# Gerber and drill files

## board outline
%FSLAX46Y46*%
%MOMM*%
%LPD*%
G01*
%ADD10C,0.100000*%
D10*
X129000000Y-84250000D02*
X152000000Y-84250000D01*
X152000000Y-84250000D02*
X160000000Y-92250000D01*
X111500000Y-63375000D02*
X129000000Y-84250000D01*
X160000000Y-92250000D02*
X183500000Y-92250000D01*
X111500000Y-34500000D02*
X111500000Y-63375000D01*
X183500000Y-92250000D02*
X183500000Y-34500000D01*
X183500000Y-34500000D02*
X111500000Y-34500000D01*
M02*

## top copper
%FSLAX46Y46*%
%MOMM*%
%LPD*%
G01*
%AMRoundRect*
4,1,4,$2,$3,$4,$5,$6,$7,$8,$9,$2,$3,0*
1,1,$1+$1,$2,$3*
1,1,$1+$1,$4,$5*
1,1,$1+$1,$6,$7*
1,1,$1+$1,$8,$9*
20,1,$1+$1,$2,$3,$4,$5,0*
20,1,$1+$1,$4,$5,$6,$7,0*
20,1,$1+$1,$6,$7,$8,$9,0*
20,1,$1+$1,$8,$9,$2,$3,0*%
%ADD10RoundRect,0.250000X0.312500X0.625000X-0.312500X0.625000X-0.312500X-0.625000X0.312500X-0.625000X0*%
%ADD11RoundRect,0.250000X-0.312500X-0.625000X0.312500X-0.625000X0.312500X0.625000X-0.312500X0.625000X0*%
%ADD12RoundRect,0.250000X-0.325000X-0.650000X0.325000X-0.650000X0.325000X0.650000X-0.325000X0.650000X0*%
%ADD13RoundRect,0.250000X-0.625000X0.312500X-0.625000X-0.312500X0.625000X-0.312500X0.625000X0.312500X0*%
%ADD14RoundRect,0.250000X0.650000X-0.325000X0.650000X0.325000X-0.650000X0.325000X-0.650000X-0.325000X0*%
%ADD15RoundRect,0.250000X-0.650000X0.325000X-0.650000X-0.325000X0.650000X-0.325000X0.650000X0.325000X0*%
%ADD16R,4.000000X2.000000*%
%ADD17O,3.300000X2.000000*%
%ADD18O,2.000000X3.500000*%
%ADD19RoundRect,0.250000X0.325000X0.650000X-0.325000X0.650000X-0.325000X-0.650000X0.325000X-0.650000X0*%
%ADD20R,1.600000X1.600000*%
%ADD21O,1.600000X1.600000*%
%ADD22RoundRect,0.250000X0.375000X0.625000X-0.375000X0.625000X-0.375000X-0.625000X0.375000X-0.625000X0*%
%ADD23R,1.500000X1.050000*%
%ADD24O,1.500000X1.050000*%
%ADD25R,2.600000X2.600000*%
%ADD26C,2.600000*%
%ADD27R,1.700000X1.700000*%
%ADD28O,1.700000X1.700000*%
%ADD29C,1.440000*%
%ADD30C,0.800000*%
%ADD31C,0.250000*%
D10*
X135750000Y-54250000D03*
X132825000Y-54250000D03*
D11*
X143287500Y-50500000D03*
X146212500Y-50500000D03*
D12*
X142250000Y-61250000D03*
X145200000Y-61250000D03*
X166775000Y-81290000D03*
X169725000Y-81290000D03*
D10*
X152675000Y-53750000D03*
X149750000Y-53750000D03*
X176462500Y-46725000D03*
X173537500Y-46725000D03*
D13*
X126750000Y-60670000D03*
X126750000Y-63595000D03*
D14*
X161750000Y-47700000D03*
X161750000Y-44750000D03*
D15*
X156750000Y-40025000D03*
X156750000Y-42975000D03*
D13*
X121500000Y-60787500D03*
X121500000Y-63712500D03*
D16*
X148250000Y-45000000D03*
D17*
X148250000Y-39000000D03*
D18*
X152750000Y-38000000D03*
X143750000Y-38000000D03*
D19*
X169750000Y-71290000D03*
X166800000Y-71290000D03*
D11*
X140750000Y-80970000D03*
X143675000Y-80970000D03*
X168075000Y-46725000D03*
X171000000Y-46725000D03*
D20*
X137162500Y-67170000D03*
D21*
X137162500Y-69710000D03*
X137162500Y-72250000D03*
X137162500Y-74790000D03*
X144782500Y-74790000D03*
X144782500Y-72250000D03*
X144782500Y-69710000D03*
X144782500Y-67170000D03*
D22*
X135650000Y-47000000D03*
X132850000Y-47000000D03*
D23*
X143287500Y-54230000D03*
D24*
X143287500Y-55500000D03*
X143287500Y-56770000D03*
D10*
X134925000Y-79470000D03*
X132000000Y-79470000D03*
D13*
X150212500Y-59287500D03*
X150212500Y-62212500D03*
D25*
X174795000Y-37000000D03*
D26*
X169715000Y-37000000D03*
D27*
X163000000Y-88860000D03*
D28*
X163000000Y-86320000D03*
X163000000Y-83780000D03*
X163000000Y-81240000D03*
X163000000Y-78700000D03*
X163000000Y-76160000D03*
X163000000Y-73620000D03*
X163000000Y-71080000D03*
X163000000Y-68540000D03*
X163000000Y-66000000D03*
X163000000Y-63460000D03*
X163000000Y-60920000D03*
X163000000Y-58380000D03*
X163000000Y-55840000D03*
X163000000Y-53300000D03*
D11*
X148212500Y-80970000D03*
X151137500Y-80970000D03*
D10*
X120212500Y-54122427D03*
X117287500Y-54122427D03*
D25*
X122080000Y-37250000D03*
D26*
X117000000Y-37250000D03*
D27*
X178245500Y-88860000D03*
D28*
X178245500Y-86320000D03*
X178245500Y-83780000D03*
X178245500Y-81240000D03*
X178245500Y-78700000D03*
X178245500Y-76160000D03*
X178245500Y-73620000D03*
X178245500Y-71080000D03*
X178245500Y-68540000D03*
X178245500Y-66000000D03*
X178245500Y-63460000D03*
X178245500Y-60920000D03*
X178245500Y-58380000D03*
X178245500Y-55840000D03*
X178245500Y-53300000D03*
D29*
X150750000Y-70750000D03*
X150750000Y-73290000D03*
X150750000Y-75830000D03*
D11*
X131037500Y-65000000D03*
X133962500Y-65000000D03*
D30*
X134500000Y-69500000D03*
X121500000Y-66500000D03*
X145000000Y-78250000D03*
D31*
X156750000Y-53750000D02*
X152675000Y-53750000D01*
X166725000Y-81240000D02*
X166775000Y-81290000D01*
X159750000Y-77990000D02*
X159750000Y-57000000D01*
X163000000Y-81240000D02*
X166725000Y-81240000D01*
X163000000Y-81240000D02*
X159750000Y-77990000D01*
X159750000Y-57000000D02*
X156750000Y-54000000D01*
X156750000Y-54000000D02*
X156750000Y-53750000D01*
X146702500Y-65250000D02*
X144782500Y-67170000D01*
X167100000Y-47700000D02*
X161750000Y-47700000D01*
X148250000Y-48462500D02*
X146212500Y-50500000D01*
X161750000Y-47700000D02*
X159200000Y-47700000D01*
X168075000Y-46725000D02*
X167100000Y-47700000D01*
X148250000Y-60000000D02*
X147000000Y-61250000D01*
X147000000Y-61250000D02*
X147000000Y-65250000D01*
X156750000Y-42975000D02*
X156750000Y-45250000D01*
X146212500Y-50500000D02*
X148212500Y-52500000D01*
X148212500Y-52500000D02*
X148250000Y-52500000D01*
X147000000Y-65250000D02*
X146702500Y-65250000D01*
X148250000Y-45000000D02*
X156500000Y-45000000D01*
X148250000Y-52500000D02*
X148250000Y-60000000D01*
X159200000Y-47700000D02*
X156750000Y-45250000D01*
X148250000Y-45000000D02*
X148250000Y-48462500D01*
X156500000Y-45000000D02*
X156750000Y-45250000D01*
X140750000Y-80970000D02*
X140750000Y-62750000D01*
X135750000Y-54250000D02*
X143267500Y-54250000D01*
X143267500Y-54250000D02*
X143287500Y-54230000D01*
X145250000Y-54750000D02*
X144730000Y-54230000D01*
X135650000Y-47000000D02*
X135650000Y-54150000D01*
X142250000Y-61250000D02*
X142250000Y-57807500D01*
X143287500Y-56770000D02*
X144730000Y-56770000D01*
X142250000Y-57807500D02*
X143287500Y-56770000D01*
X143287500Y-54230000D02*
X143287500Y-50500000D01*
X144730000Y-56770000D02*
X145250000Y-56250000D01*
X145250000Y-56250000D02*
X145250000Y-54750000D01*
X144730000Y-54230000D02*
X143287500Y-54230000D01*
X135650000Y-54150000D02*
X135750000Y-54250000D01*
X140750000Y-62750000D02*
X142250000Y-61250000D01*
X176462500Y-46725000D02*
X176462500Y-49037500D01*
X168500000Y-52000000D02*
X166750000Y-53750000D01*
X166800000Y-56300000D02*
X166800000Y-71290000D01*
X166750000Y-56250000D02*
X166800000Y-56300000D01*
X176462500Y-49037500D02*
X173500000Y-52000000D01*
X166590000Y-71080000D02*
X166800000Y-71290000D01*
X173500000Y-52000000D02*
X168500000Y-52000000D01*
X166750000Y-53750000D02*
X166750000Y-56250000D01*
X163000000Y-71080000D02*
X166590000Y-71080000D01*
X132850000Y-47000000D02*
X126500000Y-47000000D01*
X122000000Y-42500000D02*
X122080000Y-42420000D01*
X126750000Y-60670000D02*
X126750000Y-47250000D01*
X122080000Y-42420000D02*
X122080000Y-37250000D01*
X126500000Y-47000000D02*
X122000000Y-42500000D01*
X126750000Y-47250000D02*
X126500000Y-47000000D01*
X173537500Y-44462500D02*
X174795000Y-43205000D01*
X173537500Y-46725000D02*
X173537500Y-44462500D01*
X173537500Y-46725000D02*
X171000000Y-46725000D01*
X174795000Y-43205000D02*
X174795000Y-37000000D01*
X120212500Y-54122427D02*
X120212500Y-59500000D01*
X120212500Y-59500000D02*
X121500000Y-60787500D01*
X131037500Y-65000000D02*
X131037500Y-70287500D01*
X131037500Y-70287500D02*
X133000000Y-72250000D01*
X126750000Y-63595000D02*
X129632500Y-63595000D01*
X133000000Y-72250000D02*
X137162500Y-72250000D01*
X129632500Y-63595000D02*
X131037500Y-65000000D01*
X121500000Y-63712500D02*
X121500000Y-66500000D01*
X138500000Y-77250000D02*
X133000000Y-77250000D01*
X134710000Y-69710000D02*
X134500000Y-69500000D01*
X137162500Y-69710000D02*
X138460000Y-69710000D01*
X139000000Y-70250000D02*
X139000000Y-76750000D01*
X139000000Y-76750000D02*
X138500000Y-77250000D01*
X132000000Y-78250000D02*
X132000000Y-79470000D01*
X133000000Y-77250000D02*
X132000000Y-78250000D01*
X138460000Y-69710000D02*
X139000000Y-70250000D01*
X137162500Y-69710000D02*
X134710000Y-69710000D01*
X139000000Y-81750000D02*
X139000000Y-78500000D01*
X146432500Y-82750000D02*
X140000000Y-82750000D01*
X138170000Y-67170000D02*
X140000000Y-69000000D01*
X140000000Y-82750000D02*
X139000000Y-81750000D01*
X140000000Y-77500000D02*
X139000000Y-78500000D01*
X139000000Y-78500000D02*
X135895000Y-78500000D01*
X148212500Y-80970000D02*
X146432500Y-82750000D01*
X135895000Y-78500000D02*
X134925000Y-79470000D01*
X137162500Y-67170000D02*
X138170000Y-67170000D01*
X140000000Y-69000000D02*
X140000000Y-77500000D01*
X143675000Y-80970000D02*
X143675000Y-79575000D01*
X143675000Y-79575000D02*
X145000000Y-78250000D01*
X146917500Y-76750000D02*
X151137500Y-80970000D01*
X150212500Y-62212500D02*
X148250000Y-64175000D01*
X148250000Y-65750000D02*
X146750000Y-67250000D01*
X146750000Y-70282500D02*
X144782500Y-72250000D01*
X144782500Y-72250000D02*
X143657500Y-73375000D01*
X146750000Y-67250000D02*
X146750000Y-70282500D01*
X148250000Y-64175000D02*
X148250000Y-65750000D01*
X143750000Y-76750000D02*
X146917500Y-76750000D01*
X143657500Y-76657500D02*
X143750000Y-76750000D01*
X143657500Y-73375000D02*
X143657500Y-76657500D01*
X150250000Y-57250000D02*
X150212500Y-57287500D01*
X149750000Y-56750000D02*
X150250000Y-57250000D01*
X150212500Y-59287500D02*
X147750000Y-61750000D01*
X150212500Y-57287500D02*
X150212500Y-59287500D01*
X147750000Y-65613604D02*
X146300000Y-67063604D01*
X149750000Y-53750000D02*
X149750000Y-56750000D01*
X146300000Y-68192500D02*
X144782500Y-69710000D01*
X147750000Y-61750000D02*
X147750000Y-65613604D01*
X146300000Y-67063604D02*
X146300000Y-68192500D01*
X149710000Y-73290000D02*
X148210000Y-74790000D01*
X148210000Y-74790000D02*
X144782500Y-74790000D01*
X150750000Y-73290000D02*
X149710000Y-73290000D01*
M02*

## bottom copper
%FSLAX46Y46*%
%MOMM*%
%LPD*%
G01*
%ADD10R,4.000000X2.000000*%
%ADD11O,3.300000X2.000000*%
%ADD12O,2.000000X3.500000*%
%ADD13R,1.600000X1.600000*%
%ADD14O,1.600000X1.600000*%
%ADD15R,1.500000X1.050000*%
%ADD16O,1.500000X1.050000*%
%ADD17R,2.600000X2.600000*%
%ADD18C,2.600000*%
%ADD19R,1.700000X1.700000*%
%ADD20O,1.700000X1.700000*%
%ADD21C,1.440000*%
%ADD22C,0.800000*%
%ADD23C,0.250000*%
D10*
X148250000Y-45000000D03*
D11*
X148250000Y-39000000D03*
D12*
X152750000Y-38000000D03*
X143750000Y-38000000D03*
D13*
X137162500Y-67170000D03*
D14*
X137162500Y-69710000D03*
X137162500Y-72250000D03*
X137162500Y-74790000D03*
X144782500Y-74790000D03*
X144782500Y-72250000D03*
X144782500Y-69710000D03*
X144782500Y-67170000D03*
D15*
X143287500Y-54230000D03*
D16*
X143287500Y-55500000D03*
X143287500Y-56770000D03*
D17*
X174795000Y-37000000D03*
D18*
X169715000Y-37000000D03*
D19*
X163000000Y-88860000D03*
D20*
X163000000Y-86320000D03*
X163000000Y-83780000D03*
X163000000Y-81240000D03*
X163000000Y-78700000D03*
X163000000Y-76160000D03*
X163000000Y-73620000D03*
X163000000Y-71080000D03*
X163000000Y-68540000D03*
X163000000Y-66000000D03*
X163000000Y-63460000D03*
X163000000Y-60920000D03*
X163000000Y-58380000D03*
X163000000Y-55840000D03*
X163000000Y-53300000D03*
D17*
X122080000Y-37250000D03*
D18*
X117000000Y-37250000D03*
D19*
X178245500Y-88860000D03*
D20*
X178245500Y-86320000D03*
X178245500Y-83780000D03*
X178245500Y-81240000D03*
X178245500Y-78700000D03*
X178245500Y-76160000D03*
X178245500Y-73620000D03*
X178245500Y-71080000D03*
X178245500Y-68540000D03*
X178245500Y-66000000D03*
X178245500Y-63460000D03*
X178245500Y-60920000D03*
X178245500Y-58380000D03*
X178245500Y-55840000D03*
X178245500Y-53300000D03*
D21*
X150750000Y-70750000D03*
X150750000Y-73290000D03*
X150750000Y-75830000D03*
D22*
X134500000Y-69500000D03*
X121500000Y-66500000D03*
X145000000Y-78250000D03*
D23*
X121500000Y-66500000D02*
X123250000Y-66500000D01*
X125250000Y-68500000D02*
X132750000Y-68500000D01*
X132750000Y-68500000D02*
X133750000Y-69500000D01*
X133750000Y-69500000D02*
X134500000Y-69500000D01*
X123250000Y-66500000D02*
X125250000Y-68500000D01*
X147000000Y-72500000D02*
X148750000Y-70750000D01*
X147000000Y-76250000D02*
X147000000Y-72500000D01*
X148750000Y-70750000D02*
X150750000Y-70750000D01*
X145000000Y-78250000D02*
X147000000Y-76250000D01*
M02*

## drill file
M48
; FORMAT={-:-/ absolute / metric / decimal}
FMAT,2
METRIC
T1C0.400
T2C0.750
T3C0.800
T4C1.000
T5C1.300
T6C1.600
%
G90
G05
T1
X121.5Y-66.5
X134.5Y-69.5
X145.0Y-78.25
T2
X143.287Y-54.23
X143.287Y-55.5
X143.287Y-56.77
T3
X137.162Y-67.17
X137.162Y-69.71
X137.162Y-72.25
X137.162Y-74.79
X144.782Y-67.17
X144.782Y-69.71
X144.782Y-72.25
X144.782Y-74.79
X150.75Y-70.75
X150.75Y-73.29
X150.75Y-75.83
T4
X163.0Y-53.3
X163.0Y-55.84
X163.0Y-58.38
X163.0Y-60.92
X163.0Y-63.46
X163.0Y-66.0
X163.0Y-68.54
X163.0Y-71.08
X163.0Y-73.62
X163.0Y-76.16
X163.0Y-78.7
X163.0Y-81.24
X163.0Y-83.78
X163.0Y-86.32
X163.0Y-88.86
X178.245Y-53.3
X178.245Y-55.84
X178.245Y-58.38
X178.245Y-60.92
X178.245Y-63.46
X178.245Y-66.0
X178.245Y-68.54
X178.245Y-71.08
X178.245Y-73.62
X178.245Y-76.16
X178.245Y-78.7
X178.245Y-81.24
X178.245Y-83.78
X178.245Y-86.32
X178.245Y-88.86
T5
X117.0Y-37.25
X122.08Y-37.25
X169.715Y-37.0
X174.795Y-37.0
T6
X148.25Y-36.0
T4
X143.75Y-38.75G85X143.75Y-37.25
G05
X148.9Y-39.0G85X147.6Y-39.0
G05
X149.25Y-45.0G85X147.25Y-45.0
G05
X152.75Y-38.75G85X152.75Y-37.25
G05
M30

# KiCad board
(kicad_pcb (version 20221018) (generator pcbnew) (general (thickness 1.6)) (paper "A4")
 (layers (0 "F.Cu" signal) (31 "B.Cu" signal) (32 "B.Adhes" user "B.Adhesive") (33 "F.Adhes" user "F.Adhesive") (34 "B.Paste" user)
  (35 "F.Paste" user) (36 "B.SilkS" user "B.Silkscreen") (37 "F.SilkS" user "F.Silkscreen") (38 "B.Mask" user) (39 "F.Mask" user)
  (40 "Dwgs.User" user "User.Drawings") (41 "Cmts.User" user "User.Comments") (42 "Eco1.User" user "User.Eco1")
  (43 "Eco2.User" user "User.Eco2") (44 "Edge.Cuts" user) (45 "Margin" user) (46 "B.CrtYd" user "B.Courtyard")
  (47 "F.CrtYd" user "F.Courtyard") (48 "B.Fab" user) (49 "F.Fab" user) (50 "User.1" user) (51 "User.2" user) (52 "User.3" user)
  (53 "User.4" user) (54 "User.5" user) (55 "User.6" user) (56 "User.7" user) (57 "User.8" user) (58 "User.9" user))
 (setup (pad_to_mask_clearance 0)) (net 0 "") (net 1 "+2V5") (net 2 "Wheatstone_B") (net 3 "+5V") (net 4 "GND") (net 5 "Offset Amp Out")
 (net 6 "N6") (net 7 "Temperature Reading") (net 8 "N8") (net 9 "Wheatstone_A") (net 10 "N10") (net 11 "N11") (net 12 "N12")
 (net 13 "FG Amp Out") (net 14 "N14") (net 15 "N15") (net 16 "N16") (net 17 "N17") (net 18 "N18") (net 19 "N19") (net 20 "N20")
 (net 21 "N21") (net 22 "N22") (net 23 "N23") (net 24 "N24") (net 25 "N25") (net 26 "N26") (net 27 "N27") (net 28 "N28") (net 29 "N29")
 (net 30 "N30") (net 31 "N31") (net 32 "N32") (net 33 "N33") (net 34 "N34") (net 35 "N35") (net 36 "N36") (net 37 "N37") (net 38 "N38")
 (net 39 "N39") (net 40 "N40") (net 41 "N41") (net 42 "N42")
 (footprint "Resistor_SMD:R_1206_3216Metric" (layer "F.Cu") (at 134.2875 54.25 180)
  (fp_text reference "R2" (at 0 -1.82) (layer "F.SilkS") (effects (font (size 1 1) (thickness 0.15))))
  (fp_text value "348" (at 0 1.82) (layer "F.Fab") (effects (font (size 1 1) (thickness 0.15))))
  (pad "1" smd roundrect (at -1.4625 0 180) (size 1.125 1.75) (layers "F.Cu" "F.Paste" "F.Mask") (roundrect_rratio 0.222222) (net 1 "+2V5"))
  (pad "2" smd roundrect (at 1.4625 0 180) (size 1.125 1.75) (layers "F.Cu" "F.Paste" "F.Mask") (roundrect_rratio 0.222222)
   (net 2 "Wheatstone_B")))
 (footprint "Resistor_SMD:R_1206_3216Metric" (layer "F.Cu") (at 144.75 50.5)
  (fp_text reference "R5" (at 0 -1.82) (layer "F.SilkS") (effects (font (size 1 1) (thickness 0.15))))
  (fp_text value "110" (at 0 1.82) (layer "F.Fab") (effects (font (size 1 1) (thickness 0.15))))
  (pad "1" smd roundrect (at -1.4625 0) (size 1.125 1.75) (layers "F.Cu" "F.Paste" "F.Mask") (roundrect_rratio 0.222222) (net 1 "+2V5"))
  (pad "2" smd roundrect (at 1.4625 0) (size 1.125 1.75) (layers "F.Cu" "F.Paste" "F.Mask") (roundrect_rratio 0.222222) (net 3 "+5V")))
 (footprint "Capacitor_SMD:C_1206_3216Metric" (layer "F.Cu") (at 143.725 61.25)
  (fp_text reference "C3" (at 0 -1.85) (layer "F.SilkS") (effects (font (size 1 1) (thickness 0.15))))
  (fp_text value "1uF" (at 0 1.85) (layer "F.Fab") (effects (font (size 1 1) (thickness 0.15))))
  (pad "1" smd roundrect (at -1.475 0) (size 1.15 1.8) (layers "F.Cu" "F.Paste" "F.Mask") (roundrect_rratio 0.217391) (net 1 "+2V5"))
  (pad "2" smd roundrect (at 1.475 0) (size 1.15 1.8) (layers "F.Cu" "F.Paste" "F.Mask") (roundrect_rratio 0.217391) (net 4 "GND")))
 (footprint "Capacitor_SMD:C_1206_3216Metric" (layer "F.Cu") (at 168.25 81.29)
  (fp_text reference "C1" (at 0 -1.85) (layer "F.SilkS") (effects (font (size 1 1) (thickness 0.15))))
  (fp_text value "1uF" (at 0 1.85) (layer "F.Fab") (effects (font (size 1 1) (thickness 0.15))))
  (pad "1" smd roundrect (at -1.475 0) (size 1.15 1.8) (layers "F.Cu" "F.Paste" "F.Mask") (roundrect_rratio 0.217391)
   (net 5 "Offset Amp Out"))
  (pad "2" smd roundrect (at 1.475 0) (size 1.15 1.8) (layers "F.Cu" "F.Paste" "F.Mask") (roundrect_rratio 0.217391) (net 4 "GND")))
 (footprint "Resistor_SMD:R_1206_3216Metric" (layer "F.Cu") (at 151.2125 53.75 180)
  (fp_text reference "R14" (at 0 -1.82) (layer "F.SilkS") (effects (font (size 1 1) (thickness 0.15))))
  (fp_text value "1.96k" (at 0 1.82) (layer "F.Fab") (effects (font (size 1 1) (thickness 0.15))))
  (pad "1" smd roundrect (at -1.4625 0 180) (size 1.125 1.75) (layers "F.Cu" "F.Paste" "F.Mask") (roundrect_rratio 0.222222)
   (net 5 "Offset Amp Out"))
  (pad "2" smd roundrect (at 1.4625 0 180) (size 1.125 1.75) (layers "F.Cu" "F.Paste" "F.Mask") (roundrect_rratio 0.222222) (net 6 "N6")))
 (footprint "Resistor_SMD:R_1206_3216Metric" (layer "F.Cu") (at 175 46.725 180)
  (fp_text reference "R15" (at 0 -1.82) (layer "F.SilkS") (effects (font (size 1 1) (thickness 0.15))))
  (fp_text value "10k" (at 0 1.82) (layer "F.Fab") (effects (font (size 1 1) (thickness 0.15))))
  (pad "1" smd roundrect (at -1.4625 0 180) (size 1.125 1.75) (layers "F.Cu" "F.Paste" "F.Mask") (roundrect_rratio 0.222222)
   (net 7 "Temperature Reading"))
  (pad "2" smd roundrect (at 1.4625 0 180) (size 1.125 1.75) (layers "F.Cu" "F.Paste" "F.Mask") (roundrect_rratio 0.222222) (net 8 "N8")))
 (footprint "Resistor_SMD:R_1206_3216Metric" (layer "F.Cu") (at 126.75 62.1325 -90)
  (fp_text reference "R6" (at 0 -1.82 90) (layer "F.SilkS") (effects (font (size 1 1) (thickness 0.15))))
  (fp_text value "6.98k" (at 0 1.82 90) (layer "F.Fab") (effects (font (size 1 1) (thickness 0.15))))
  (pad "1" smd roundrect (at -1.4625 0 270) (size 1.125 1.75) (layers "F.Cu" "F.Paste" "F.Mask") (roundrect_rratio 0.222222)
   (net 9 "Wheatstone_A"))
  (pad "2" smd roundrect (at 1.4625 0 270) (size 1.125 1.75) (layers "F.Cu" "F.Paste" "F.Mask") (roundrect_rratio 0.222222) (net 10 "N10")))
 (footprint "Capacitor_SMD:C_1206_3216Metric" (layer "F.Cu") (at 161.75 46.225 90)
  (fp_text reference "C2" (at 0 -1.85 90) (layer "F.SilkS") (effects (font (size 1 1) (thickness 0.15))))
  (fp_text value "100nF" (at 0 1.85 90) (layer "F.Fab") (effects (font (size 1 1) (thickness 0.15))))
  (pad "1" smd roundrect (at -1.475 0 90) (size 1.15 1.8) (layers "F.Cu" "F.Paste" "F.Mask") (roundrect_rratio 0.217391) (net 3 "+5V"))
  (pad "2" smd roundrect (at 1.475 0 90) (size 1.15 1.8) (layers "F.Cu" "F.Paste" "F.Mask") (roundrect_rratio 0.217391) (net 4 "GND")))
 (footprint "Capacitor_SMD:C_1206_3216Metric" (layer "F.Cu") (at 156.75 41.5 -90)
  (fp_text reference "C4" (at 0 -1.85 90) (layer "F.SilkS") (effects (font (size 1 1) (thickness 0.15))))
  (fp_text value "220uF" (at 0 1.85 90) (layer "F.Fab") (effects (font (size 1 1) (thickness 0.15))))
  (pad "1" smd roundrect (at -1.475 0 270) (size 1.15 1.8) (layers "F.Cu" "F.Paste" "F.Mask") (roundrect_rratio 0.217391) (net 4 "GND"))
  (pad "2" smd roundrect (at 1.475 0 270) (size 1.15 1.8) (layers "F.Cu" "F.Paste" "F.Mask") (roundrect_rratio 0.217391) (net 3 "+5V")))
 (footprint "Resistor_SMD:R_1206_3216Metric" (layer "F.Cu") (at 121.5 62.25 -90)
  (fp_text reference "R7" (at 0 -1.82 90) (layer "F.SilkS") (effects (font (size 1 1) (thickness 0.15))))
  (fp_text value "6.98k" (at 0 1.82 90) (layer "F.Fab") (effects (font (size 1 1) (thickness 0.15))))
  (pad "1" smd roundrect (at -1.4625 0 270) (size 1.125 1.75) (layers "F.Cu" "F.Paste" "F.Mask") (roundrect_rratio 0.222222)
   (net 2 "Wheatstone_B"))
  (pad "2" smd roundrect (at 1.4625 0 270) (size 1.125 1.75) (layers "F.Cu" "F.Paste" "F.Mask") (roundrect_rratio 0.222222) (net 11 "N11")))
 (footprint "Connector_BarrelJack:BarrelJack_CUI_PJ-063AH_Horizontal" (layer "F.Cu") (at 148.25 45 180)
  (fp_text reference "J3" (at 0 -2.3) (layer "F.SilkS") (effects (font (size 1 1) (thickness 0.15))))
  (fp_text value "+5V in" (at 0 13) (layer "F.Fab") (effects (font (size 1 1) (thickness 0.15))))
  (pad "" np_thru_hole circle (at 0 9 180) (size 1.6 1.6) (drill 1.6) (layers "*.Cu" "*.Mask"))
  (pad "1" thru_hole rect (at 0 0 180) (size 4 2) (drill oval 3 1) (layers "*.Cu" "*.Mask") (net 3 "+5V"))
  (pad "2" thru_hole oval (at 0 6 180) (size 3.3 2) (drill oval 2.3 1) (layers "*.Cu" "*.Mask") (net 4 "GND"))
  (pad "MP" thru_hole oval (at -4.5 7 180) (size 2 3.5) (drill oval 1 2.5) (layers "*.Cu" "*.Mask"))
  (pad "MP" thru_hole oval (at 4.5 7 180) (size 2 3.5) (drill oval 1 2.5) (layers "*.Cu" "*.Mask")))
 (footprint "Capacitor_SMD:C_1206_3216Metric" (layer "F.Cu") (at 168.275 71.29 180)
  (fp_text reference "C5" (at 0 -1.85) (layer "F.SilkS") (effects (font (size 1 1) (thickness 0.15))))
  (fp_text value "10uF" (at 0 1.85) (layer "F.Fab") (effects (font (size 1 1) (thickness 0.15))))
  (pad "1" smd roundrect (at -1.475 0 180) (size 1.15 1.8) (layers "F.Cu" "F.Paste" "F.Mask") (roundrect_rratio 0.217391) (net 4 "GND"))
  (pad "2" smd roundrect (at 1.475 0 180) (size 1.15 1.8) (layers "F.Cu" "F.Paste" "F.Mask") (roundrect_rratio 0.217391)
   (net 7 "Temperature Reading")))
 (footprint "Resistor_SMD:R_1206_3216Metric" (layer "F.Cu") (at 142.2125 80.97)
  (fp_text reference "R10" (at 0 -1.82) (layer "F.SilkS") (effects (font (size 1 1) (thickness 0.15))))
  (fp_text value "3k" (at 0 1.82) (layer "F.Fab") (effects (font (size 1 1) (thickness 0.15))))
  (pad "1" smd roundrect (at -1.4625 0) (size 1.125 1.75) (layers "F.Cu" "F.Paste" "F.Mask") (roundrect_rratio 0.222222) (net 1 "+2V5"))
  (pad "2" smd roundrect (at 1.4625 0) (size 1.125 1.75) (layers "F.Cu" "F.Paste" "F.Mask") (roundrect_rratio 0.222222) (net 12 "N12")))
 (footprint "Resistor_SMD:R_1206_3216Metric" (layer "F.Cu") (at 169.5375 46.725)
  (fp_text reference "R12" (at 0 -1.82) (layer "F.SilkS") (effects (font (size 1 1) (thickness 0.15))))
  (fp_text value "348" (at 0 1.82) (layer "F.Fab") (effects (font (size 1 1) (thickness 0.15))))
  (pad "1" smd roundrect (at -1.4625 0) (size 1.125 1.75) (layers "F.Cu" "F.Paste" "F.Mask") (roundrect_rratio 0.222222) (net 3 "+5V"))
  (pad "2" smd roundrect (at 1.4625 0) (size 1.125 1.75) (layers "F.Cu" "F.Paste" "F.Mask") (roundrect_rratio 0.222222) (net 8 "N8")))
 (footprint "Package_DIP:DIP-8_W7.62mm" (layer "F.Cu") (at 137.1625 67.17)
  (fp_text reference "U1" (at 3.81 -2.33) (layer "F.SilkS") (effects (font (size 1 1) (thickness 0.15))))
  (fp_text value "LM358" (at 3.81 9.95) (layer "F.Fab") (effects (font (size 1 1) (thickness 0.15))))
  (pad "1" thru_hole rect (at 0 0) (size 1.6 1.6) (drill 0.8) (layers "*.Cu" "*.Mask") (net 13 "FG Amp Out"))
  (pad "2" thru_hole oval (at 0 2.54) (size 1.6 1.6) (drill 0.8) (layers "*.Cu" "*.Mask") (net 11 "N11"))
  (pad "3" thru_hole oval (at 0 5.08) (size 1.6 1.6) (drill 0.8) (layers "*.Cu" "*.Mask") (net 10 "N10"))
  (pad "4" thru_hole oval (at 0 7.62) (size 1.6 1.6) (drill 0.8) (layers "*.Cu" "*.Mask") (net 4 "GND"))
  (pad "5" thru_hole oval (at 7.62 7.62) (size 1.6 1.6) (drill 0.8) (layers "*.Cu" "*.Mask") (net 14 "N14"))
  (pad "6" thru_hole oval (at 7.62 5.08) (size 1.6 1.6) (drill 0.8) (layers "*.Cu" "*.Mask") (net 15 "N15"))
  (pad "7" thru_hole oval (at 7.62 2.54) (size 1.6 1.6) (drill 0.8) (layers "*.Cu" "*.Mask") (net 6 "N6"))
  (pad "8" thru_hole oval (at 7.62 0) (size 1.6 1.6) (drill 0.8) (layers "*.Cu" "*.Mask") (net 3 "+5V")))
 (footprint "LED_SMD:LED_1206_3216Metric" (layer "F.Cu") (at 134.25 47 180)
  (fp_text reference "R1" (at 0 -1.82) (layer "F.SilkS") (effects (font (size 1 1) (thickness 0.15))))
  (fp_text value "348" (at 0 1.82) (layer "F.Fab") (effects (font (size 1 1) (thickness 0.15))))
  (pad "1" smd roundrect (at -1.4 0 180) (size 1.25 1.75) (layers "F.Cu" "F.Paste" "F.Mask") (roundrect_rratio 0.2) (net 1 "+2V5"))
  (pad "2" smd roundrect (at 1.4 0 180) (size 1.25 1.75) (layers "F.Cu" "F.Paste" "F.Mask") (roundrect_rratio 0.2) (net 9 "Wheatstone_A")))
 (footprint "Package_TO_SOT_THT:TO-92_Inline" (layer "F.Cu") (at 143.2875 54.23 -90)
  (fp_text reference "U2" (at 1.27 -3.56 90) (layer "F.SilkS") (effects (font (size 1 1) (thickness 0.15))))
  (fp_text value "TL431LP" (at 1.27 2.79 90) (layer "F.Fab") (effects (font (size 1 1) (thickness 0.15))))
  (pad "1" thru_hole rect (at 0 0 270) (size 1.05 1.5) (drill 0.75) (layers "*.Cu" "*.Mask") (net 1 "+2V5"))
  (pad "2" thru_hole oval (at 1.27 0 270) (size 1.05 1.5) (drill 0.75) (layers "*.Cu" "*.Mask") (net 4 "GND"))
  (pad "3" thru_hole oval (at 2.54 0 270) (size 1.05 1.5) (drill 0.75) (layers "*.Cu" "*.Mask") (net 1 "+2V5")))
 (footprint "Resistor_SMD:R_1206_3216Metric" (layer "F.Cu") (at 133.4625 79.47 180)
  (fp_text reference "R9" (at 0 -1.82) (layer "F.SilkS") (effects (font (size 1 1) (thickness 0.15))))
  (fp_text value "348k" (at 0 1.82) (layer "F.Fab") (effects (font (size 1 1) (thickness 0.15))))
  (pad "1" smd roundrect (at -1.4625 0 180) (size 1.125 1.75) (layers "F.Cu" "F.Paste" "F.Mask") (roundrect_rratio 0.222222)
   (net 13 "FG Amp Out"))
  (pad "2" smd roundrect (at 1.4625 0 180) (size 1.125 1.75) (layers "F.Cu" "F.Paste" "F.Mask") (roundrect_rratio 0.222222) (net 11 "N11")))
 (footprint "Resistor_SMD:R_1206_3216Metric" (layer "F.Cu") (at 150.2125 60.75 -90)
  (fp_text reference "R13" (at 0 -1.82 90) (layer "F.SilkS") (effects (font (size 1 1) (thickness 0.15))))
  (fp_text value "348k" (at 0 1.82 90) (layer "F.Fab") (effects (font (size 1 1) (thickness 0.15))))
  (pad "1" smd roundrect (at -1.4625 0 270) (size 1.125 1.75) (layers "F.Cu" "F.Paste" "F.Mask") (roundrect_rratio 0.222222) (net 6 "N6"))
  (pad "2" smd roundrect (at 1.4625 0 270) (size 1.125 1.75) (layers "F.Cu" "F.Paste" "F.Mask") (roundrect_rratio 0.222222) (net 15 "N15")))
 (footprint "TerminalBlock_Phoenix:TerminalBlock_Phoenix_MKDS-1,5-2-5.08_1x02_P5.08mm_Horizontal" (layer "F.Cu") (at 174.795 37 180)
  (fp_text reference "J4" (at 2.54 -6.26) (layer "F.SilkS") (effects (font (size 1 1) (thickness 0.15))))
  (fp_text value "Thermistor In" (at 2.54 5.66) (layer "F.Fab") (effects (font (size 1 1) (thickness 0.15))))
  (pad "1" thru_hole rect (at 0 0 180) (size 2.6 2.6) (drill 1.3) (layers "*.Cu" "*.Mask") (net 8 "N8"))
  (pad "2" thru_hole circle (at 5.08 0 180) (size 2.6 2.6) (drill 1.3) (layers "*.Cu" "*.Mask") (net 4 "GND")))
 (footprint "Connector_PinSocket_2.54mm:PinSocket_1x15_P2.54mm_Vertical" (layer "F.Cu") (at 163 88.86 180)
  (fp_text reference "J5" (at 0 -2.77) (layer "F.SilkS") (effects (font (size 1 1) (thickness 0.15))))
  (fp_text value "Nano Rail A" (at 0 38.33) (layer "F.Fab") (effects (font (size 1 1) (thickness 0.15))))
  (pad "1" thru_hole rect (at 0 0 180) (size 1.7 1.7) (drill 1) (layers "*.Cu" "*.Mask") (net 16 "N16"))
  (pad "2" thru_hole oval (at 0 2.54 180) (size 1.7 1.7) (drill 1) (layers "*.Cu" "*.Mask") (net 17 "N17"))
  (pad "3" thru_hole oval (at 0 5.08 180) (size 1.7 1.7) (drill 1) (layers "*.Cu" "*.Mask") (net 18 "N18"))
  (pad "4" thru_hole oval (at 0 7.62 180) (size 1.7 1.7) (drill 1) (layers "*.Cu" "*.Mask") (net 5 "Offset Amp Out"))
  (pad "5" thru_hole oval (at 0 10.16 180) (size 1.7 1.7) (drill 1) (layers "*.Cu" "*.Mask") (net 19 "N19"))
  (pad "6" thru_hole oval (at 0 12.7 180) (size 1.7 1.7) (drill 1) (layers "*.Cu" "*.Mask") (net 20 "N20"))
  (pad "7" thru_hole oval (at 0 15.24 180) (size 1.7 1.7) (drill 1) (layers "*.Cu" "*.Mask") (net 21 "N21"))
  (pad "8" thru_hole oval (at 0 17.78 180) (size 1.7 1.7) (drill 1) (layers "*.Cu" "*.Mask") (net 7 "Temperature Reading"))
  (pad "9" thru_hole oval (at 0 20.32 180) (size 1.7 1.7) (drill 1) (layers "*.Cu" "*.Mask") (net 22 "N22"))
  (pad "10" thru_hole oval (at 0 22.86 180) (size 1.7 1.7) (drill 1) (layers "*.Cu" "*.Mask") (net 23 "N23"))
  (pad "11" thru_hole oval (at 0 25.4 180) (size 1.7 1.7) (drill 1) (layers "*.Cu" "*.Mask") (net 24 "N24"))
  (pad "12" thru_hole oval (at 0 27.94 180) (size 1.7 1.7) (drill 1) (layers "*.Cu" "*.Mask") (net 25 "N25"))
  (pad "13" thru_hole oval (at 0 30.48 180) (size 1.7 1.7) (drill 1) (layers "*.Cu" "*.Mask") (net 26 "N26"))
  (pad "14" thru_hole oval (at 0 33.02 180) (size 1.7 1.7) (drill 1) (layers "*.Cu" "*.Mask") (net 4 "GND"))
  (pad "15" thru_hole oval (at 0 35.56 180) (size 1.7 1.7) (drill 1) (layers "*.Cu" "*.Mask") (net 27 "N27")))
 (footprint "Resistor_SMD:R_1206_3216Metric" (layer "F.Cu") (at 149.675 80.97)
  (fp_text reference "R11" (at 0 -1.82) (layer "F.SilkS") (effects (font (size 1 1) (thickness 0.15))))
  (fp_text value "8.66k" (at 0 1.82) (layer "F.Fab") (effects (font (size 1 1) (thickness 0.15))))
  (pad "1" smd roundrect (at -1.4625 0) (size 1.125 1.75) (layers "F.Cu" "F.Paste" "F.Mask") (roundrect_rratio 0.222222)
   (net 13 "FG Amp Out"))
  (pad "2" smd roundrect (at 1.4625 0) (size 1.125 1.75) (layers "F.Cu" "F.Paste" "F.Mask") (roundrect_rratio 0.222222) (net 15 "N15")))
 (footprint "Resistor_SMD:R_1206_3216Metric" (layer "F.Cu") (at 118.75 54.122427 180)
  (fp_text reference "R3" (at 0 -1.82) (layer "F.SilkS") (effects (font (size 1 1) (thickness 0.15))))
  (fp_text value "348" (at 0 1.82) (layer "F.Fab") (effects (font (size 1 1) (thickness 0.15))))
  (pad "1" smd roundrect (at -1.4625 0 180) (size 1.125 1.75) (layers "F.Cu" "F.Paste" "F.Mask") (roundrect_rratio 0.222222)
   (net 2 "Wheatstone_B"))
  (pad "2" smd roundrect (at 1.4625 0 180) (size 1.125 1.75) (layers "F.Cu" "F.Paste" "F.Mask") (roundrect_rratio 0.222222) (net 4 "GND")))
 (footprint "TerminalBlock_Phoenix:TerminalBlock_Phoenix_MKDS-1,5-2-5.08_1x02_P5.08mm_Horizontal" (layer "F.Cu") (at 122.08 37.25 180)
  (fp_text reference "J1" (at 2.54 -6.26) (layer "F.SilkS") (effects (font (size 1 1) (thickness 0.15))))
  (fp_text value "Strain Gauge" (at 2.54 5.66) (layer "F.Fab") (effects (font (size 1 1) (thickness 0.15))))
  (pad "1" thru_hole rect (at 0 0 180) (size 2.6 2.6) (drill 1.3) (layers "*.Cu" "*.Mask") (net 9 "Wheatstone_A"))
  (pad "2" thru_hole circle (at 5.08 0 180) (size 2.6 2.6) (drill 1.3) (layers "*.Cu" "*.Mask") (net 4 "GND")))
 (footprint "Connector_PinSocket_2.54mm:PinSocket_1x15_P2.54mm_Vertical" (layer "F.Cu") (at 178.2455 88.86 180)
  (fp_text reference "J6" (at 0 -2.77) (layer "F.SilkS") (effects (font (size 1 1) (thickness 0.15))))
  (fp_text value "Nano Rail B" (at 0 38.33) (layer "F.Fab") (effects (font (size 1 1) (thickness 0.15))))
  (pad "1" thru_hole rect (at 0 0 180) (size 1.7 1.7) (drill 1) (layers "*.Cu" "*.Mask") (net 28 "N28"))
  (pad "2" thru_hole oval (at 0 2.54 180) (size 1.7 1.7) (drill 1) (layers "*.Cu" "*.Mask") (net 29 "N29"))
  (pad "3" thru_hole oval (at 0 5.08 180) (size 1.7 1.7) (drill 1) (layers "*.Cu" "*.Mask") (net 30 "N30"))
  (pad "4" thru_hole oval (at 0 7.62 180) (size 1.7 1.7) (drill 1) (layers "*.Cu" "*.Mask") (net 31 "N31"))
  (pad "5" thru_hole oval (at 0 10.16 180) (size 1.7 1.7) (drill 1) (layers "*.Cu" "*.Mask") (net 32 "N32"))
  (pad "6" thru_hole oval (at 0 12.7 180) (size 1.7 1.7) (drill 1) (layers "*.Cu" "*.Mask") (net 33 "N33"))
  (pad "7" thru_hole oval (at 0 15.24 180) (size 1.7 1.7) (drill 1) (layers "*.Cu" "*.Mask") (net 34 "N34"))
  (pad "8" thru_hole oval (at 0 17.78 180) (size 1.7 1.7) (drill 1) (layers "*.Cu" "*.Mask") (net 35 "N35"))
  (pad "9" thru_hole oval (at 0 20.32 180) (size 1.7 1.7) (drill 1) (layers "*.Cu" "*.Mask") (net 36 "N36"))
  (pad "10" thru_hole oval (at 0 22.86 180) (size 1.7 1.7) (drill 1) (layers "*.Cu" "*.Mask") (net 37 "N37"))
  (pad "11" thru_hole oval (at 0 25.4 180) (size 1.7 1.7) (drill 1) (layers "*.Cu" "*.Mask") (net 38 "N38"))
  (pad "12" thru_hole oval (at 0 27.94 180) (size 1.7 1.7) (drill 1) (layers "*.Cu" "*.Mask") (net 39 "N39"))
  (pad "13" thru_hole oval (at 0 30.48 180) (size 1.7 1.7) (drill 1) (layers "*.Cu" "*.Mask") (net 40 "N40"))
  (pad "14" thru_hole oval (at 0 33.02 180) (size 1.7 1.7) (drill 1) (layers "*.Cu" "*.Mask") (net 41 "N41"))
  (pad "15" thru_hole oval (at 0 35.56 180) (size 1.7 1.7) (drill 1) (layers "*.Cu" "*.Mask") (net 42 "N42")))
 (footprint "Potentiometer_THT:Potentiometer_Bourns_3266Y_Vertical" (layer "F.Cu") (at 150.75 70.75 90)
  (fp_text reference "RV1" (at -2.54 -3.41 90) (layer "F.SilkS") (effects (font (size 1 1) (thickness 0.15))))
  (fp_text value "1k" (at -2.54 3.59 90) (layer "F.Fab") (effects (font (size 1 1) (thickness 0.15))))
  (pad "1" thru_hole circle (at 0 0 90) (size 1.44 1.44) (drill 0.8) (layers "*.Cu" "*.Mask") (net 12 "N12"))
  (pad "2" thru_hole circle (at -2.54 0 90) (size 1.44 1.44) (drill 0.8) (layers "*.Cu" "*.Mask") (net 14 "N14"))
  (pad "3" thru_hole circle (at -5.08 0 90) (size 1.44 1.44) (drill 0.8) (layers "*.Cu" "*.Mask") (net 4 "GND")))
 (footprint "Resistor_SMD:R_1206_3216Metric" (layer "F.Cu") (at 132.5 65)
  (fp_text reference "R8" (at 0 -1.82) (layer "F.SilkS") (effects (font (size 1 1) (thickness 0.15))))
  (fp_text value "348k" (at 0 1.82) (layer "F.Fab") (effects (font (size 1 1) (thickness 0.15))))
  (pad "1" smd roundrect (at -1.4625 0) (size 1.125 1.75) (layers "F.Cu" "F.Paste" "F.Mask") (roundrect_rratio 0.222222) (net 10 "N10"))
  (pad "2" smd roundrect (at 1.4625 0) (size 1.125 1.75) (layers "F.Cu" "F.Paste" "F.Mask") (roundrect_rratio 0.222222) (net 4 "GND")))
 (gr_line (start 129 84.25) (end 152 84.25) (stroke (width 0.1) (type default)) (layer "Edge.Cuts"))
 (gr_line (start 152 84.25) (end 160 92.25) (stroke (width 0.1) (type default)) (layer "Edge.Cuts"))
 (gr_line (start 111.5 63.375) (end 129 84.25) (stroke (width 0.1) (type default)) (layer "Edge.Cuts"))
 (gr_line (start 160 92.25) (end 183.5 92.25) (stroke (width 0.1) (type default)) (layer "Edge.Cuts"))
 (gr_line (start 111.5 34.5) (end 111.5 63.375) (stroke (width 0.1) (type default)) (layer "Edge.Cuts"))
 (gr_line (start 183.5 92.25) (end 183.5 34.5) (stroke (width 0.1) (type default)) (layer "Edge.Cuts"))
 (gr_line (start 183.5 34.5) (end 111.5 34.5) (stroke (width 0.1) (type default)) (layer "Edge.Cuts"))
 (segment (start 156.75 53.75) (end 152.675 53.75) (width 0.25) (layer "F.Cu") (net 5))
 (segment (start 166.725 81.24) (end 166.775 81.29) (width 0.25) (layer "F.Cu") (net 5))
 (segment (start 159.75 77.99) (end 159.75 57) (width 0.25) (layer "F.Cu") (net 5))
 (segment (start 163 81.24) (end 166.725 81.24) (width 0.25) (layer "F.Cu") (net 5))
 (segment (start 163 81.24) (end 159.75 77.99) (width 0.25) (layer "F.Cu") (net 5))
 (segment (start 159.75 57) (end 156.75 54) (width 0.25) (layer "F.Cu") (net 5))
 (segment (start 156.75 54) (end 156.75 53.75) (width 0.25) (layer "F.Cu") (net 5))
 (segment (start 146.7025 65.25) (end 144.7825 67.17) (width 0.25) (layer "F.Cu") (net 3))
 (segment (start 167.1 47.7) (end 161.75 47.7) (width 0.25) (layer "F.Cu") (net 3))
 (segment (start 148.25 48.4625) (end 146.2125 50.5) (width 0.25) (layer "F.Cu") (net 3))
 (segment (start 161.75 47.7) (end 159.2 47.7) (width 0.25) (layer "F.Cu") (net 3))
 (segment (start 168.075 46.725) (end 167.1 47.7) (width 0.25) (layer "F.Cu") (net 3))
 (segment (start 148.25 60) (end 147 61.25) (width 0.25) (layer "F.Cu") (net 3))
 (segment (start 147 61.25) (end 147 65.25) (width 0.25) (layer "F.Cu") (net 3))
 (segment (start 156.75 42.975) (end 156.75 45.25) (width 0.25) (layer "F.Cu") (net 3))
 (segment (start 146.2125 50.5) (end 148.2125 52.5) (width 0.25) (layer "F.Cu") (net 3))
 (segment (start 148.2125 52.5) (end 148.25 52.5) (width 0.25) (layer "F.Cu") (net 3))
 (segment (start 147 65.25) (end 146.7025 65.25) (width 0.25) (layer "F.Cu") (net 3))
 (segment (start 148.25 45) (end 156.5 45) (width 0.25) (layer "F.Cu") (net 3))
 (segment (start 148.25 52.5) (end 148.25 60) (width 0.25) (layer "F.Cu") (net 3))
 (segment (start 159.2 47.7) (end 156.75 45.25) (width 0.25) (layer "F.Cu") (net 3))
 (segment (start 148.25 45) (end 148.25 48.4625) (width 0.25) (layer "F.Cu") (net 3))
 (segment (start 156.5 45) (end 156.75 45.25) (width 0.25) (layer "F.Cu") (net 3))
 (segment (start 140.75 80.97) (end 140.75 62.75) (width 0.25) (layer "F.Cu") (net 1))
 (segment (start 135.75 54.25) (end 143.2675 54.25) (width 0.25) (layer "F.Cu") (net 1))
 (segment (start 143.2675 54.25) (end 143.2875 54.23) (width 0.25) (layer "F.Cu") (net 1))
 (segment (start 145.25 54.75) (end 144.73 54.23) (width 0.25) (layer "F.Cu") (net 1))
 (segment (start 135.65 47) (end 135.65 54.15) (width 0.25) (layer "F.Cu") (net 1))
 (segment (start 142.25 61.25) (end 142.25 57.8075) (width 0.25) (layer "F.Cu") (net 1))
 (segment (start 143.2875 56.77) (end 144.73 56.77) (width 0.25) (layer "F.Cu") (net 1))
 (segment (start 142.25 57.8075) (end 143.2875 56.77) (width 0.25) (layer "F.Cu") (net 1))
 (segment (start 143.2875 54.23) (end 143.2875 50.5) (width 0.25) (layer "F.Cu") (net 1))
 (segment (start 144.73 56.77) (end 145.25 56.25) (width 0.25) (layer "F.Cu") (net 1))
 (segment (start 145.25 56.25) (end 145.25 54.75) (width 0.25) (layer "F.Cu") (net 1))
 (segment (start 144.73 54.23) (end 143.2875 54.23) (width 0.25) (layer "F.Cu") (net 1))
 (segment (start 135.65 54.15) (end 135.75 54.25) (width 0.25) (layer "F.Cu") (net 1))
 (segment (start 140.75 62.75) (end 142.25 61.25) (width 0.25) (layer "F.Cu") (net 1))
 (segment (start 176.4625 46.725) (end 176.4625 49.0375) (width 0.25) (layer "F.Cu") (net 7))
 (segment (start 168.5 52) (end 166.75 53.75) (width 0.25) (layer "F.Cu") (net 7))
 (segment (start 166.8 56.3) (end 166.8 71.29) (width 0.25) (layer "F.Cu") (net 7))
 (segment (start 166.75 56.25) (end 166.8 56.3) (width 0.25) (layer "F.Cu") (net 7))
 (segment (start 176.4625 49.0375) (end 173.5 52) (width 0.25) (layer "F.Cu") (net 7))
 (segment (start 166.59 71.08) (end 166.8 71.29) (width 0.25) (layer "F.Cu") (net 7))
 (segment (start 173.5 52) (end 168.5 52) (width 0.25) (layer "F.Cu") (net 7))
 (segment (start 166.75 53.75) (end 166.75 56.25) (width 0.25) (layer "F.Cu") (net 7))
 (segment (start 163 71.08) (end 166.59 71.08) (width 0.25) (layer "F.Cu") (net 7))
 (segment (start 132.85 47) (end 126.5 47) (width 0.25) (layer "F.Cu") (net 9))
 (segment (start 122 42.5) (end 122.08 42.42) (width 0.25) (layer "F.Cu") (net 9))
 (segment (start 126.75 60.67) (end 126.75 47.25) (width 0.25) (layer "F.Cu") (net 9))
 (segment (start 122.08 42.42) (end 122.08 37.25) (width 0.25) (layer "F.Cu") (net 9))
 (segment (start 126.5 47) (end 122 42.5) (width 0.25) (layer "F.Cu") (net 9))
 (segment (start 126.75 47.25) (end 126.5 47) (width 0.25) (layer "F.Cu") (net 9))
 (segment (start 173.5375 44.4625) (end 174.795 43.205) (width 0.25) (layer "F.Cu") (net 8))
 (segment (start 173.5375 46.725) (end 173.5375 44.4625) (width 0.25) (layer "F.Cu") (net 8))
 (segment (start 173.5375 46.725) (end 171 46.725) (width 0.25) (layer "F.Cu") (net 8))
 (segment (start 174.795 43.205) (end 174.795 37) (width 0.25) (layer "F.Cu") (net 8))
 (segment (start 120.2125 54.122427) (end 120.2125 59.5) (width 0.25) (layer "F.Cu") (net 2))
 (segment (start 120.2125 59.5) (end 121.5 60.7875) (width 0.25) (layer "F.Cu") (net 2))
 (segment (start 131.0375 65) (end 131.0375 70.2875) (width 0.25) (layer "F.Cu") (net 10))
 (segment (start 131.0375 70.2875) (end 133 72.25) (width 0.25) (layer "F.Cu") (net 10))
 (segment (start 126.75 63.595) (end 129.6325 63.595) (width 0.25) (layer "F.Cu") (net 10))
 (segment (start 133 72.25) (end 137.1625 72.25) (width 0.25) (layer "F.Cu") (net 10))
 (segment (start 129.6325 63.595) (end 131.0375 65) (width 0.25) (layer "F.Cu") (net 10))
 (segment (start 121.5 63.7125) (end 121.5 66.5) (width 0.25) (layer "F.Cu") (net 11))
 (segment (start 138.5 77.25) (end 133 77.25) (width 0.25) (layer "F.Cu") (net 11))
 (segment (start 134.71 69.71) (end 134.5 69.5) (width 0.25) (layer "F.Cu") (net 11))
 (segment (start 137.1625 69.71) (end 138.46 69.71) (width 0.25) (layer "F.Cu") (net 11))
 (segment (start 139 70.25) (end 139 76.75) (width 0.25) (layer "F.Cu") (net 11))
 (segment (start 139 76.75) (end 138.5 77.25) (width 0.25) (layer "F.Cu") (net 11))
 (segment (start 132 78.25) (end 132 79.47) (width 0.25) (layer "F.Cu") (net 11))
 (segment (start 133 77.25) (end 132 78.25) (width 0.25) (layer "F.Cu") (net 11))
 (segment (start 138.46 69.71) (end 139 70.25) (width 0.25) (layer "F.Cu") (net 11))
 (segment (start 137.1625 69.71) (end 134.71 69.71) (width 0.25) (layer "F.Cu") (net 11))
 (via (at 134.5 69.5) (size 0.8) (drill 0.4) (layers "F.Cu" "B.Cu") (free) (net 11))
 (via (at 121.5 66.5) (size 0.8) (drill 0.4) (layers "F.Cu" "B.Cu") (free) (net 11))
 (segment (start 121.5 66.5) (end 123.25 66.5) (width 0.25) (layer "B.Cu") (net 11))
 (segment (start 125.25 68.5) (end 132.75 68.5) (width 0.25) (layer "B.Cu") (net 11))
 (segment (start 132.75 68.5) (end 133.75 69.5) (width 0.25) (layer "B.Cu") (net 11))
 (segment (start 133.75 69.5) (end 134.5 69.5) (width 0.25) (layer "B.Cu") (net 11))
 (segment (start 123.25 66.5) (end 125.25 68.5) (width 0.25) (layer "B.Cu") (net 11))
 (segment (start 139 81.75) (end 139 78.5) (width 0.25) (layer "F.Cu") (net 13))
 (segment (start 146.4325 82.75) (end 140 82.75) (width 0.25) (layer "F.Cu") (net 13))
 (segment (start 138.17 67.17) (end 140 69) (width 0.25) (layer "F.Cu") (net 13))
 (segment (start 140 82.75) (end 139 81.75) (width 0.25) (layer "F.Cu") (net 13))
 (segment (start 140 77.5) (end 139 78.5) (width 0.25) (layer "F.Cu") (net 13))
 (segment (start 139 78.5) (end 135.895 78.5) (width 0.25) (layer "F.Cu") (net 13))
 (segment (start 148.2125 80.97) (end 146.4325 82.75) (width 0.25) (layer "F.Cu") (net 13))
 (segment (start 135.895 78.5) (end 134.925 79.47) (width 0.25) (layer "F.Cu") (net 13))
 (segment (start 137.1625 67.17) (end 138.17 67.17) (width 0.25) (layer "F.Cu") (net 13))
 (segment (start 140 69) (end 140 77.5) (width 0.25) (layer "F.Cu") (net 13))
 (segment (start 143.675 80.97) (end 143.675 79.575) (width 0.25) (layer "F.Cu") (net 12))
 (segment (start 143.675 79.575) (end 145 78.25) (width 0.25) (layer "F.Cu") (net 12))
 (via (at 145 78.25) (size 0.8) (drill 0.4) (layers "F.Cu" "B.Cu") (free) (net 12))
 (segment (start 147 72.5) (end 148.75 70.75) (width 0.25) (layer "B.Cu") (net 12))
 (segment (start 147 76.25) (end 147 72.5) (width 0.25) (layer "B.Cu") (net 12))
 (segment (start 148.75 70.75) (end 150.75 70.75) (width 0.25) (layer "B.Cu") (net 12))
 (segment (start 145 78.25) (end 147 76.25) (width 0.25) (layer "B.Cu") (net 12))
 (segment (start 146.9175 76.75) (end 151.1375 80.97) (width 0.25) (layer "F.Cu") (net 15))
 (segment (start 150.2125 62.2125) (end 148.25 64.175) (width 0.25) (layer "F.Cu") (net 15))
 (segment (start 148.25 65.75) (end 146.75 67.25) (width 0.25) (layer "F.Cu") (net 15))
 (segment (start 146.75 70.2825) (end 144.7825 72.25) (width 0.25) (layer "F.Cu") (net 15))
 (segment (start 144.7825 72.25) (end 143.6575 73.375) (width 0.25) (layer "F.Cu") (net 15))
 (segment (start 146.75 67.25) (end 146.75 70.2825) (width 0.25) (layer "F.Cu") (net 15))
 (segment (start 148.25 64.175) (end 148.25 65.75) (width 0.25) (layer "F.Cu") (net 15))
 (segment (start 143.75 76.75) (end 146.9175 76.75) (width 0.25) (layer "F.Cu") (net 15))
 (segment (start 143.6575 76.6575) (end 143.75 76.75) (width 0.25) (layer "F.Cu") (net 15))
 (segment (start 143.6575 73.375) (end 143.6575 76.6575) (width 0.25) (layer "F.Cu") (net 15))
 (segment (start 150.25 57.25) (end 150.2125 57.2875) (width 0.25) (layer "F.Cu") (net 6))
 (segment (start 149.75 56.75) (end 150.25 57.25) (width 0.25) (layer "F.Cu") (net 6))
 (segment (start 150.2125 59.2875) (end 147.75 61.75) (width 0.25) (layer "F.Cu") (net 6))
 (segment (start 150.2125 57.2875) (end 150.2125 59.2875) (width 0.25) (layer "F.Cu") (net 6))
 (segment (start 147.75 65.613604) (end 146.3 67.063604) (width 0.25) (layer "F.Cu") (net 6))
 (segment (start 149.75 53.75) (end 149.75 56.75) (width 0.25) (layer "F.Cu") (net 6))
 (segment (start 146.3 68.1925) (end 144.7825 69.71) (width 0.25) (layer "F.Cu") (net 6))
 (segment (start 147.75 61.75) (end 147.75 65.613604) (width 0.25) (layer "F.Cu") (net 6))
 (segment (start 146.3 67.063604) (end 146.3 68.1925) (width 0.25) (layer "F.Cu") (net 6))
 (segment (start 149.71 73.29) (end 148.21 74.79) (width 0.25) (layer "F.Cu") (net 14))
 (segment (start 148.21 74.79) (end 144.7825 74.79) (width 0.25) (layer "F.Cu") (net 14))
 (segment (start 150.75 73.29) (end 149.71 73.29) (width 0.25) (layer "F.Cu") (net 14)))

